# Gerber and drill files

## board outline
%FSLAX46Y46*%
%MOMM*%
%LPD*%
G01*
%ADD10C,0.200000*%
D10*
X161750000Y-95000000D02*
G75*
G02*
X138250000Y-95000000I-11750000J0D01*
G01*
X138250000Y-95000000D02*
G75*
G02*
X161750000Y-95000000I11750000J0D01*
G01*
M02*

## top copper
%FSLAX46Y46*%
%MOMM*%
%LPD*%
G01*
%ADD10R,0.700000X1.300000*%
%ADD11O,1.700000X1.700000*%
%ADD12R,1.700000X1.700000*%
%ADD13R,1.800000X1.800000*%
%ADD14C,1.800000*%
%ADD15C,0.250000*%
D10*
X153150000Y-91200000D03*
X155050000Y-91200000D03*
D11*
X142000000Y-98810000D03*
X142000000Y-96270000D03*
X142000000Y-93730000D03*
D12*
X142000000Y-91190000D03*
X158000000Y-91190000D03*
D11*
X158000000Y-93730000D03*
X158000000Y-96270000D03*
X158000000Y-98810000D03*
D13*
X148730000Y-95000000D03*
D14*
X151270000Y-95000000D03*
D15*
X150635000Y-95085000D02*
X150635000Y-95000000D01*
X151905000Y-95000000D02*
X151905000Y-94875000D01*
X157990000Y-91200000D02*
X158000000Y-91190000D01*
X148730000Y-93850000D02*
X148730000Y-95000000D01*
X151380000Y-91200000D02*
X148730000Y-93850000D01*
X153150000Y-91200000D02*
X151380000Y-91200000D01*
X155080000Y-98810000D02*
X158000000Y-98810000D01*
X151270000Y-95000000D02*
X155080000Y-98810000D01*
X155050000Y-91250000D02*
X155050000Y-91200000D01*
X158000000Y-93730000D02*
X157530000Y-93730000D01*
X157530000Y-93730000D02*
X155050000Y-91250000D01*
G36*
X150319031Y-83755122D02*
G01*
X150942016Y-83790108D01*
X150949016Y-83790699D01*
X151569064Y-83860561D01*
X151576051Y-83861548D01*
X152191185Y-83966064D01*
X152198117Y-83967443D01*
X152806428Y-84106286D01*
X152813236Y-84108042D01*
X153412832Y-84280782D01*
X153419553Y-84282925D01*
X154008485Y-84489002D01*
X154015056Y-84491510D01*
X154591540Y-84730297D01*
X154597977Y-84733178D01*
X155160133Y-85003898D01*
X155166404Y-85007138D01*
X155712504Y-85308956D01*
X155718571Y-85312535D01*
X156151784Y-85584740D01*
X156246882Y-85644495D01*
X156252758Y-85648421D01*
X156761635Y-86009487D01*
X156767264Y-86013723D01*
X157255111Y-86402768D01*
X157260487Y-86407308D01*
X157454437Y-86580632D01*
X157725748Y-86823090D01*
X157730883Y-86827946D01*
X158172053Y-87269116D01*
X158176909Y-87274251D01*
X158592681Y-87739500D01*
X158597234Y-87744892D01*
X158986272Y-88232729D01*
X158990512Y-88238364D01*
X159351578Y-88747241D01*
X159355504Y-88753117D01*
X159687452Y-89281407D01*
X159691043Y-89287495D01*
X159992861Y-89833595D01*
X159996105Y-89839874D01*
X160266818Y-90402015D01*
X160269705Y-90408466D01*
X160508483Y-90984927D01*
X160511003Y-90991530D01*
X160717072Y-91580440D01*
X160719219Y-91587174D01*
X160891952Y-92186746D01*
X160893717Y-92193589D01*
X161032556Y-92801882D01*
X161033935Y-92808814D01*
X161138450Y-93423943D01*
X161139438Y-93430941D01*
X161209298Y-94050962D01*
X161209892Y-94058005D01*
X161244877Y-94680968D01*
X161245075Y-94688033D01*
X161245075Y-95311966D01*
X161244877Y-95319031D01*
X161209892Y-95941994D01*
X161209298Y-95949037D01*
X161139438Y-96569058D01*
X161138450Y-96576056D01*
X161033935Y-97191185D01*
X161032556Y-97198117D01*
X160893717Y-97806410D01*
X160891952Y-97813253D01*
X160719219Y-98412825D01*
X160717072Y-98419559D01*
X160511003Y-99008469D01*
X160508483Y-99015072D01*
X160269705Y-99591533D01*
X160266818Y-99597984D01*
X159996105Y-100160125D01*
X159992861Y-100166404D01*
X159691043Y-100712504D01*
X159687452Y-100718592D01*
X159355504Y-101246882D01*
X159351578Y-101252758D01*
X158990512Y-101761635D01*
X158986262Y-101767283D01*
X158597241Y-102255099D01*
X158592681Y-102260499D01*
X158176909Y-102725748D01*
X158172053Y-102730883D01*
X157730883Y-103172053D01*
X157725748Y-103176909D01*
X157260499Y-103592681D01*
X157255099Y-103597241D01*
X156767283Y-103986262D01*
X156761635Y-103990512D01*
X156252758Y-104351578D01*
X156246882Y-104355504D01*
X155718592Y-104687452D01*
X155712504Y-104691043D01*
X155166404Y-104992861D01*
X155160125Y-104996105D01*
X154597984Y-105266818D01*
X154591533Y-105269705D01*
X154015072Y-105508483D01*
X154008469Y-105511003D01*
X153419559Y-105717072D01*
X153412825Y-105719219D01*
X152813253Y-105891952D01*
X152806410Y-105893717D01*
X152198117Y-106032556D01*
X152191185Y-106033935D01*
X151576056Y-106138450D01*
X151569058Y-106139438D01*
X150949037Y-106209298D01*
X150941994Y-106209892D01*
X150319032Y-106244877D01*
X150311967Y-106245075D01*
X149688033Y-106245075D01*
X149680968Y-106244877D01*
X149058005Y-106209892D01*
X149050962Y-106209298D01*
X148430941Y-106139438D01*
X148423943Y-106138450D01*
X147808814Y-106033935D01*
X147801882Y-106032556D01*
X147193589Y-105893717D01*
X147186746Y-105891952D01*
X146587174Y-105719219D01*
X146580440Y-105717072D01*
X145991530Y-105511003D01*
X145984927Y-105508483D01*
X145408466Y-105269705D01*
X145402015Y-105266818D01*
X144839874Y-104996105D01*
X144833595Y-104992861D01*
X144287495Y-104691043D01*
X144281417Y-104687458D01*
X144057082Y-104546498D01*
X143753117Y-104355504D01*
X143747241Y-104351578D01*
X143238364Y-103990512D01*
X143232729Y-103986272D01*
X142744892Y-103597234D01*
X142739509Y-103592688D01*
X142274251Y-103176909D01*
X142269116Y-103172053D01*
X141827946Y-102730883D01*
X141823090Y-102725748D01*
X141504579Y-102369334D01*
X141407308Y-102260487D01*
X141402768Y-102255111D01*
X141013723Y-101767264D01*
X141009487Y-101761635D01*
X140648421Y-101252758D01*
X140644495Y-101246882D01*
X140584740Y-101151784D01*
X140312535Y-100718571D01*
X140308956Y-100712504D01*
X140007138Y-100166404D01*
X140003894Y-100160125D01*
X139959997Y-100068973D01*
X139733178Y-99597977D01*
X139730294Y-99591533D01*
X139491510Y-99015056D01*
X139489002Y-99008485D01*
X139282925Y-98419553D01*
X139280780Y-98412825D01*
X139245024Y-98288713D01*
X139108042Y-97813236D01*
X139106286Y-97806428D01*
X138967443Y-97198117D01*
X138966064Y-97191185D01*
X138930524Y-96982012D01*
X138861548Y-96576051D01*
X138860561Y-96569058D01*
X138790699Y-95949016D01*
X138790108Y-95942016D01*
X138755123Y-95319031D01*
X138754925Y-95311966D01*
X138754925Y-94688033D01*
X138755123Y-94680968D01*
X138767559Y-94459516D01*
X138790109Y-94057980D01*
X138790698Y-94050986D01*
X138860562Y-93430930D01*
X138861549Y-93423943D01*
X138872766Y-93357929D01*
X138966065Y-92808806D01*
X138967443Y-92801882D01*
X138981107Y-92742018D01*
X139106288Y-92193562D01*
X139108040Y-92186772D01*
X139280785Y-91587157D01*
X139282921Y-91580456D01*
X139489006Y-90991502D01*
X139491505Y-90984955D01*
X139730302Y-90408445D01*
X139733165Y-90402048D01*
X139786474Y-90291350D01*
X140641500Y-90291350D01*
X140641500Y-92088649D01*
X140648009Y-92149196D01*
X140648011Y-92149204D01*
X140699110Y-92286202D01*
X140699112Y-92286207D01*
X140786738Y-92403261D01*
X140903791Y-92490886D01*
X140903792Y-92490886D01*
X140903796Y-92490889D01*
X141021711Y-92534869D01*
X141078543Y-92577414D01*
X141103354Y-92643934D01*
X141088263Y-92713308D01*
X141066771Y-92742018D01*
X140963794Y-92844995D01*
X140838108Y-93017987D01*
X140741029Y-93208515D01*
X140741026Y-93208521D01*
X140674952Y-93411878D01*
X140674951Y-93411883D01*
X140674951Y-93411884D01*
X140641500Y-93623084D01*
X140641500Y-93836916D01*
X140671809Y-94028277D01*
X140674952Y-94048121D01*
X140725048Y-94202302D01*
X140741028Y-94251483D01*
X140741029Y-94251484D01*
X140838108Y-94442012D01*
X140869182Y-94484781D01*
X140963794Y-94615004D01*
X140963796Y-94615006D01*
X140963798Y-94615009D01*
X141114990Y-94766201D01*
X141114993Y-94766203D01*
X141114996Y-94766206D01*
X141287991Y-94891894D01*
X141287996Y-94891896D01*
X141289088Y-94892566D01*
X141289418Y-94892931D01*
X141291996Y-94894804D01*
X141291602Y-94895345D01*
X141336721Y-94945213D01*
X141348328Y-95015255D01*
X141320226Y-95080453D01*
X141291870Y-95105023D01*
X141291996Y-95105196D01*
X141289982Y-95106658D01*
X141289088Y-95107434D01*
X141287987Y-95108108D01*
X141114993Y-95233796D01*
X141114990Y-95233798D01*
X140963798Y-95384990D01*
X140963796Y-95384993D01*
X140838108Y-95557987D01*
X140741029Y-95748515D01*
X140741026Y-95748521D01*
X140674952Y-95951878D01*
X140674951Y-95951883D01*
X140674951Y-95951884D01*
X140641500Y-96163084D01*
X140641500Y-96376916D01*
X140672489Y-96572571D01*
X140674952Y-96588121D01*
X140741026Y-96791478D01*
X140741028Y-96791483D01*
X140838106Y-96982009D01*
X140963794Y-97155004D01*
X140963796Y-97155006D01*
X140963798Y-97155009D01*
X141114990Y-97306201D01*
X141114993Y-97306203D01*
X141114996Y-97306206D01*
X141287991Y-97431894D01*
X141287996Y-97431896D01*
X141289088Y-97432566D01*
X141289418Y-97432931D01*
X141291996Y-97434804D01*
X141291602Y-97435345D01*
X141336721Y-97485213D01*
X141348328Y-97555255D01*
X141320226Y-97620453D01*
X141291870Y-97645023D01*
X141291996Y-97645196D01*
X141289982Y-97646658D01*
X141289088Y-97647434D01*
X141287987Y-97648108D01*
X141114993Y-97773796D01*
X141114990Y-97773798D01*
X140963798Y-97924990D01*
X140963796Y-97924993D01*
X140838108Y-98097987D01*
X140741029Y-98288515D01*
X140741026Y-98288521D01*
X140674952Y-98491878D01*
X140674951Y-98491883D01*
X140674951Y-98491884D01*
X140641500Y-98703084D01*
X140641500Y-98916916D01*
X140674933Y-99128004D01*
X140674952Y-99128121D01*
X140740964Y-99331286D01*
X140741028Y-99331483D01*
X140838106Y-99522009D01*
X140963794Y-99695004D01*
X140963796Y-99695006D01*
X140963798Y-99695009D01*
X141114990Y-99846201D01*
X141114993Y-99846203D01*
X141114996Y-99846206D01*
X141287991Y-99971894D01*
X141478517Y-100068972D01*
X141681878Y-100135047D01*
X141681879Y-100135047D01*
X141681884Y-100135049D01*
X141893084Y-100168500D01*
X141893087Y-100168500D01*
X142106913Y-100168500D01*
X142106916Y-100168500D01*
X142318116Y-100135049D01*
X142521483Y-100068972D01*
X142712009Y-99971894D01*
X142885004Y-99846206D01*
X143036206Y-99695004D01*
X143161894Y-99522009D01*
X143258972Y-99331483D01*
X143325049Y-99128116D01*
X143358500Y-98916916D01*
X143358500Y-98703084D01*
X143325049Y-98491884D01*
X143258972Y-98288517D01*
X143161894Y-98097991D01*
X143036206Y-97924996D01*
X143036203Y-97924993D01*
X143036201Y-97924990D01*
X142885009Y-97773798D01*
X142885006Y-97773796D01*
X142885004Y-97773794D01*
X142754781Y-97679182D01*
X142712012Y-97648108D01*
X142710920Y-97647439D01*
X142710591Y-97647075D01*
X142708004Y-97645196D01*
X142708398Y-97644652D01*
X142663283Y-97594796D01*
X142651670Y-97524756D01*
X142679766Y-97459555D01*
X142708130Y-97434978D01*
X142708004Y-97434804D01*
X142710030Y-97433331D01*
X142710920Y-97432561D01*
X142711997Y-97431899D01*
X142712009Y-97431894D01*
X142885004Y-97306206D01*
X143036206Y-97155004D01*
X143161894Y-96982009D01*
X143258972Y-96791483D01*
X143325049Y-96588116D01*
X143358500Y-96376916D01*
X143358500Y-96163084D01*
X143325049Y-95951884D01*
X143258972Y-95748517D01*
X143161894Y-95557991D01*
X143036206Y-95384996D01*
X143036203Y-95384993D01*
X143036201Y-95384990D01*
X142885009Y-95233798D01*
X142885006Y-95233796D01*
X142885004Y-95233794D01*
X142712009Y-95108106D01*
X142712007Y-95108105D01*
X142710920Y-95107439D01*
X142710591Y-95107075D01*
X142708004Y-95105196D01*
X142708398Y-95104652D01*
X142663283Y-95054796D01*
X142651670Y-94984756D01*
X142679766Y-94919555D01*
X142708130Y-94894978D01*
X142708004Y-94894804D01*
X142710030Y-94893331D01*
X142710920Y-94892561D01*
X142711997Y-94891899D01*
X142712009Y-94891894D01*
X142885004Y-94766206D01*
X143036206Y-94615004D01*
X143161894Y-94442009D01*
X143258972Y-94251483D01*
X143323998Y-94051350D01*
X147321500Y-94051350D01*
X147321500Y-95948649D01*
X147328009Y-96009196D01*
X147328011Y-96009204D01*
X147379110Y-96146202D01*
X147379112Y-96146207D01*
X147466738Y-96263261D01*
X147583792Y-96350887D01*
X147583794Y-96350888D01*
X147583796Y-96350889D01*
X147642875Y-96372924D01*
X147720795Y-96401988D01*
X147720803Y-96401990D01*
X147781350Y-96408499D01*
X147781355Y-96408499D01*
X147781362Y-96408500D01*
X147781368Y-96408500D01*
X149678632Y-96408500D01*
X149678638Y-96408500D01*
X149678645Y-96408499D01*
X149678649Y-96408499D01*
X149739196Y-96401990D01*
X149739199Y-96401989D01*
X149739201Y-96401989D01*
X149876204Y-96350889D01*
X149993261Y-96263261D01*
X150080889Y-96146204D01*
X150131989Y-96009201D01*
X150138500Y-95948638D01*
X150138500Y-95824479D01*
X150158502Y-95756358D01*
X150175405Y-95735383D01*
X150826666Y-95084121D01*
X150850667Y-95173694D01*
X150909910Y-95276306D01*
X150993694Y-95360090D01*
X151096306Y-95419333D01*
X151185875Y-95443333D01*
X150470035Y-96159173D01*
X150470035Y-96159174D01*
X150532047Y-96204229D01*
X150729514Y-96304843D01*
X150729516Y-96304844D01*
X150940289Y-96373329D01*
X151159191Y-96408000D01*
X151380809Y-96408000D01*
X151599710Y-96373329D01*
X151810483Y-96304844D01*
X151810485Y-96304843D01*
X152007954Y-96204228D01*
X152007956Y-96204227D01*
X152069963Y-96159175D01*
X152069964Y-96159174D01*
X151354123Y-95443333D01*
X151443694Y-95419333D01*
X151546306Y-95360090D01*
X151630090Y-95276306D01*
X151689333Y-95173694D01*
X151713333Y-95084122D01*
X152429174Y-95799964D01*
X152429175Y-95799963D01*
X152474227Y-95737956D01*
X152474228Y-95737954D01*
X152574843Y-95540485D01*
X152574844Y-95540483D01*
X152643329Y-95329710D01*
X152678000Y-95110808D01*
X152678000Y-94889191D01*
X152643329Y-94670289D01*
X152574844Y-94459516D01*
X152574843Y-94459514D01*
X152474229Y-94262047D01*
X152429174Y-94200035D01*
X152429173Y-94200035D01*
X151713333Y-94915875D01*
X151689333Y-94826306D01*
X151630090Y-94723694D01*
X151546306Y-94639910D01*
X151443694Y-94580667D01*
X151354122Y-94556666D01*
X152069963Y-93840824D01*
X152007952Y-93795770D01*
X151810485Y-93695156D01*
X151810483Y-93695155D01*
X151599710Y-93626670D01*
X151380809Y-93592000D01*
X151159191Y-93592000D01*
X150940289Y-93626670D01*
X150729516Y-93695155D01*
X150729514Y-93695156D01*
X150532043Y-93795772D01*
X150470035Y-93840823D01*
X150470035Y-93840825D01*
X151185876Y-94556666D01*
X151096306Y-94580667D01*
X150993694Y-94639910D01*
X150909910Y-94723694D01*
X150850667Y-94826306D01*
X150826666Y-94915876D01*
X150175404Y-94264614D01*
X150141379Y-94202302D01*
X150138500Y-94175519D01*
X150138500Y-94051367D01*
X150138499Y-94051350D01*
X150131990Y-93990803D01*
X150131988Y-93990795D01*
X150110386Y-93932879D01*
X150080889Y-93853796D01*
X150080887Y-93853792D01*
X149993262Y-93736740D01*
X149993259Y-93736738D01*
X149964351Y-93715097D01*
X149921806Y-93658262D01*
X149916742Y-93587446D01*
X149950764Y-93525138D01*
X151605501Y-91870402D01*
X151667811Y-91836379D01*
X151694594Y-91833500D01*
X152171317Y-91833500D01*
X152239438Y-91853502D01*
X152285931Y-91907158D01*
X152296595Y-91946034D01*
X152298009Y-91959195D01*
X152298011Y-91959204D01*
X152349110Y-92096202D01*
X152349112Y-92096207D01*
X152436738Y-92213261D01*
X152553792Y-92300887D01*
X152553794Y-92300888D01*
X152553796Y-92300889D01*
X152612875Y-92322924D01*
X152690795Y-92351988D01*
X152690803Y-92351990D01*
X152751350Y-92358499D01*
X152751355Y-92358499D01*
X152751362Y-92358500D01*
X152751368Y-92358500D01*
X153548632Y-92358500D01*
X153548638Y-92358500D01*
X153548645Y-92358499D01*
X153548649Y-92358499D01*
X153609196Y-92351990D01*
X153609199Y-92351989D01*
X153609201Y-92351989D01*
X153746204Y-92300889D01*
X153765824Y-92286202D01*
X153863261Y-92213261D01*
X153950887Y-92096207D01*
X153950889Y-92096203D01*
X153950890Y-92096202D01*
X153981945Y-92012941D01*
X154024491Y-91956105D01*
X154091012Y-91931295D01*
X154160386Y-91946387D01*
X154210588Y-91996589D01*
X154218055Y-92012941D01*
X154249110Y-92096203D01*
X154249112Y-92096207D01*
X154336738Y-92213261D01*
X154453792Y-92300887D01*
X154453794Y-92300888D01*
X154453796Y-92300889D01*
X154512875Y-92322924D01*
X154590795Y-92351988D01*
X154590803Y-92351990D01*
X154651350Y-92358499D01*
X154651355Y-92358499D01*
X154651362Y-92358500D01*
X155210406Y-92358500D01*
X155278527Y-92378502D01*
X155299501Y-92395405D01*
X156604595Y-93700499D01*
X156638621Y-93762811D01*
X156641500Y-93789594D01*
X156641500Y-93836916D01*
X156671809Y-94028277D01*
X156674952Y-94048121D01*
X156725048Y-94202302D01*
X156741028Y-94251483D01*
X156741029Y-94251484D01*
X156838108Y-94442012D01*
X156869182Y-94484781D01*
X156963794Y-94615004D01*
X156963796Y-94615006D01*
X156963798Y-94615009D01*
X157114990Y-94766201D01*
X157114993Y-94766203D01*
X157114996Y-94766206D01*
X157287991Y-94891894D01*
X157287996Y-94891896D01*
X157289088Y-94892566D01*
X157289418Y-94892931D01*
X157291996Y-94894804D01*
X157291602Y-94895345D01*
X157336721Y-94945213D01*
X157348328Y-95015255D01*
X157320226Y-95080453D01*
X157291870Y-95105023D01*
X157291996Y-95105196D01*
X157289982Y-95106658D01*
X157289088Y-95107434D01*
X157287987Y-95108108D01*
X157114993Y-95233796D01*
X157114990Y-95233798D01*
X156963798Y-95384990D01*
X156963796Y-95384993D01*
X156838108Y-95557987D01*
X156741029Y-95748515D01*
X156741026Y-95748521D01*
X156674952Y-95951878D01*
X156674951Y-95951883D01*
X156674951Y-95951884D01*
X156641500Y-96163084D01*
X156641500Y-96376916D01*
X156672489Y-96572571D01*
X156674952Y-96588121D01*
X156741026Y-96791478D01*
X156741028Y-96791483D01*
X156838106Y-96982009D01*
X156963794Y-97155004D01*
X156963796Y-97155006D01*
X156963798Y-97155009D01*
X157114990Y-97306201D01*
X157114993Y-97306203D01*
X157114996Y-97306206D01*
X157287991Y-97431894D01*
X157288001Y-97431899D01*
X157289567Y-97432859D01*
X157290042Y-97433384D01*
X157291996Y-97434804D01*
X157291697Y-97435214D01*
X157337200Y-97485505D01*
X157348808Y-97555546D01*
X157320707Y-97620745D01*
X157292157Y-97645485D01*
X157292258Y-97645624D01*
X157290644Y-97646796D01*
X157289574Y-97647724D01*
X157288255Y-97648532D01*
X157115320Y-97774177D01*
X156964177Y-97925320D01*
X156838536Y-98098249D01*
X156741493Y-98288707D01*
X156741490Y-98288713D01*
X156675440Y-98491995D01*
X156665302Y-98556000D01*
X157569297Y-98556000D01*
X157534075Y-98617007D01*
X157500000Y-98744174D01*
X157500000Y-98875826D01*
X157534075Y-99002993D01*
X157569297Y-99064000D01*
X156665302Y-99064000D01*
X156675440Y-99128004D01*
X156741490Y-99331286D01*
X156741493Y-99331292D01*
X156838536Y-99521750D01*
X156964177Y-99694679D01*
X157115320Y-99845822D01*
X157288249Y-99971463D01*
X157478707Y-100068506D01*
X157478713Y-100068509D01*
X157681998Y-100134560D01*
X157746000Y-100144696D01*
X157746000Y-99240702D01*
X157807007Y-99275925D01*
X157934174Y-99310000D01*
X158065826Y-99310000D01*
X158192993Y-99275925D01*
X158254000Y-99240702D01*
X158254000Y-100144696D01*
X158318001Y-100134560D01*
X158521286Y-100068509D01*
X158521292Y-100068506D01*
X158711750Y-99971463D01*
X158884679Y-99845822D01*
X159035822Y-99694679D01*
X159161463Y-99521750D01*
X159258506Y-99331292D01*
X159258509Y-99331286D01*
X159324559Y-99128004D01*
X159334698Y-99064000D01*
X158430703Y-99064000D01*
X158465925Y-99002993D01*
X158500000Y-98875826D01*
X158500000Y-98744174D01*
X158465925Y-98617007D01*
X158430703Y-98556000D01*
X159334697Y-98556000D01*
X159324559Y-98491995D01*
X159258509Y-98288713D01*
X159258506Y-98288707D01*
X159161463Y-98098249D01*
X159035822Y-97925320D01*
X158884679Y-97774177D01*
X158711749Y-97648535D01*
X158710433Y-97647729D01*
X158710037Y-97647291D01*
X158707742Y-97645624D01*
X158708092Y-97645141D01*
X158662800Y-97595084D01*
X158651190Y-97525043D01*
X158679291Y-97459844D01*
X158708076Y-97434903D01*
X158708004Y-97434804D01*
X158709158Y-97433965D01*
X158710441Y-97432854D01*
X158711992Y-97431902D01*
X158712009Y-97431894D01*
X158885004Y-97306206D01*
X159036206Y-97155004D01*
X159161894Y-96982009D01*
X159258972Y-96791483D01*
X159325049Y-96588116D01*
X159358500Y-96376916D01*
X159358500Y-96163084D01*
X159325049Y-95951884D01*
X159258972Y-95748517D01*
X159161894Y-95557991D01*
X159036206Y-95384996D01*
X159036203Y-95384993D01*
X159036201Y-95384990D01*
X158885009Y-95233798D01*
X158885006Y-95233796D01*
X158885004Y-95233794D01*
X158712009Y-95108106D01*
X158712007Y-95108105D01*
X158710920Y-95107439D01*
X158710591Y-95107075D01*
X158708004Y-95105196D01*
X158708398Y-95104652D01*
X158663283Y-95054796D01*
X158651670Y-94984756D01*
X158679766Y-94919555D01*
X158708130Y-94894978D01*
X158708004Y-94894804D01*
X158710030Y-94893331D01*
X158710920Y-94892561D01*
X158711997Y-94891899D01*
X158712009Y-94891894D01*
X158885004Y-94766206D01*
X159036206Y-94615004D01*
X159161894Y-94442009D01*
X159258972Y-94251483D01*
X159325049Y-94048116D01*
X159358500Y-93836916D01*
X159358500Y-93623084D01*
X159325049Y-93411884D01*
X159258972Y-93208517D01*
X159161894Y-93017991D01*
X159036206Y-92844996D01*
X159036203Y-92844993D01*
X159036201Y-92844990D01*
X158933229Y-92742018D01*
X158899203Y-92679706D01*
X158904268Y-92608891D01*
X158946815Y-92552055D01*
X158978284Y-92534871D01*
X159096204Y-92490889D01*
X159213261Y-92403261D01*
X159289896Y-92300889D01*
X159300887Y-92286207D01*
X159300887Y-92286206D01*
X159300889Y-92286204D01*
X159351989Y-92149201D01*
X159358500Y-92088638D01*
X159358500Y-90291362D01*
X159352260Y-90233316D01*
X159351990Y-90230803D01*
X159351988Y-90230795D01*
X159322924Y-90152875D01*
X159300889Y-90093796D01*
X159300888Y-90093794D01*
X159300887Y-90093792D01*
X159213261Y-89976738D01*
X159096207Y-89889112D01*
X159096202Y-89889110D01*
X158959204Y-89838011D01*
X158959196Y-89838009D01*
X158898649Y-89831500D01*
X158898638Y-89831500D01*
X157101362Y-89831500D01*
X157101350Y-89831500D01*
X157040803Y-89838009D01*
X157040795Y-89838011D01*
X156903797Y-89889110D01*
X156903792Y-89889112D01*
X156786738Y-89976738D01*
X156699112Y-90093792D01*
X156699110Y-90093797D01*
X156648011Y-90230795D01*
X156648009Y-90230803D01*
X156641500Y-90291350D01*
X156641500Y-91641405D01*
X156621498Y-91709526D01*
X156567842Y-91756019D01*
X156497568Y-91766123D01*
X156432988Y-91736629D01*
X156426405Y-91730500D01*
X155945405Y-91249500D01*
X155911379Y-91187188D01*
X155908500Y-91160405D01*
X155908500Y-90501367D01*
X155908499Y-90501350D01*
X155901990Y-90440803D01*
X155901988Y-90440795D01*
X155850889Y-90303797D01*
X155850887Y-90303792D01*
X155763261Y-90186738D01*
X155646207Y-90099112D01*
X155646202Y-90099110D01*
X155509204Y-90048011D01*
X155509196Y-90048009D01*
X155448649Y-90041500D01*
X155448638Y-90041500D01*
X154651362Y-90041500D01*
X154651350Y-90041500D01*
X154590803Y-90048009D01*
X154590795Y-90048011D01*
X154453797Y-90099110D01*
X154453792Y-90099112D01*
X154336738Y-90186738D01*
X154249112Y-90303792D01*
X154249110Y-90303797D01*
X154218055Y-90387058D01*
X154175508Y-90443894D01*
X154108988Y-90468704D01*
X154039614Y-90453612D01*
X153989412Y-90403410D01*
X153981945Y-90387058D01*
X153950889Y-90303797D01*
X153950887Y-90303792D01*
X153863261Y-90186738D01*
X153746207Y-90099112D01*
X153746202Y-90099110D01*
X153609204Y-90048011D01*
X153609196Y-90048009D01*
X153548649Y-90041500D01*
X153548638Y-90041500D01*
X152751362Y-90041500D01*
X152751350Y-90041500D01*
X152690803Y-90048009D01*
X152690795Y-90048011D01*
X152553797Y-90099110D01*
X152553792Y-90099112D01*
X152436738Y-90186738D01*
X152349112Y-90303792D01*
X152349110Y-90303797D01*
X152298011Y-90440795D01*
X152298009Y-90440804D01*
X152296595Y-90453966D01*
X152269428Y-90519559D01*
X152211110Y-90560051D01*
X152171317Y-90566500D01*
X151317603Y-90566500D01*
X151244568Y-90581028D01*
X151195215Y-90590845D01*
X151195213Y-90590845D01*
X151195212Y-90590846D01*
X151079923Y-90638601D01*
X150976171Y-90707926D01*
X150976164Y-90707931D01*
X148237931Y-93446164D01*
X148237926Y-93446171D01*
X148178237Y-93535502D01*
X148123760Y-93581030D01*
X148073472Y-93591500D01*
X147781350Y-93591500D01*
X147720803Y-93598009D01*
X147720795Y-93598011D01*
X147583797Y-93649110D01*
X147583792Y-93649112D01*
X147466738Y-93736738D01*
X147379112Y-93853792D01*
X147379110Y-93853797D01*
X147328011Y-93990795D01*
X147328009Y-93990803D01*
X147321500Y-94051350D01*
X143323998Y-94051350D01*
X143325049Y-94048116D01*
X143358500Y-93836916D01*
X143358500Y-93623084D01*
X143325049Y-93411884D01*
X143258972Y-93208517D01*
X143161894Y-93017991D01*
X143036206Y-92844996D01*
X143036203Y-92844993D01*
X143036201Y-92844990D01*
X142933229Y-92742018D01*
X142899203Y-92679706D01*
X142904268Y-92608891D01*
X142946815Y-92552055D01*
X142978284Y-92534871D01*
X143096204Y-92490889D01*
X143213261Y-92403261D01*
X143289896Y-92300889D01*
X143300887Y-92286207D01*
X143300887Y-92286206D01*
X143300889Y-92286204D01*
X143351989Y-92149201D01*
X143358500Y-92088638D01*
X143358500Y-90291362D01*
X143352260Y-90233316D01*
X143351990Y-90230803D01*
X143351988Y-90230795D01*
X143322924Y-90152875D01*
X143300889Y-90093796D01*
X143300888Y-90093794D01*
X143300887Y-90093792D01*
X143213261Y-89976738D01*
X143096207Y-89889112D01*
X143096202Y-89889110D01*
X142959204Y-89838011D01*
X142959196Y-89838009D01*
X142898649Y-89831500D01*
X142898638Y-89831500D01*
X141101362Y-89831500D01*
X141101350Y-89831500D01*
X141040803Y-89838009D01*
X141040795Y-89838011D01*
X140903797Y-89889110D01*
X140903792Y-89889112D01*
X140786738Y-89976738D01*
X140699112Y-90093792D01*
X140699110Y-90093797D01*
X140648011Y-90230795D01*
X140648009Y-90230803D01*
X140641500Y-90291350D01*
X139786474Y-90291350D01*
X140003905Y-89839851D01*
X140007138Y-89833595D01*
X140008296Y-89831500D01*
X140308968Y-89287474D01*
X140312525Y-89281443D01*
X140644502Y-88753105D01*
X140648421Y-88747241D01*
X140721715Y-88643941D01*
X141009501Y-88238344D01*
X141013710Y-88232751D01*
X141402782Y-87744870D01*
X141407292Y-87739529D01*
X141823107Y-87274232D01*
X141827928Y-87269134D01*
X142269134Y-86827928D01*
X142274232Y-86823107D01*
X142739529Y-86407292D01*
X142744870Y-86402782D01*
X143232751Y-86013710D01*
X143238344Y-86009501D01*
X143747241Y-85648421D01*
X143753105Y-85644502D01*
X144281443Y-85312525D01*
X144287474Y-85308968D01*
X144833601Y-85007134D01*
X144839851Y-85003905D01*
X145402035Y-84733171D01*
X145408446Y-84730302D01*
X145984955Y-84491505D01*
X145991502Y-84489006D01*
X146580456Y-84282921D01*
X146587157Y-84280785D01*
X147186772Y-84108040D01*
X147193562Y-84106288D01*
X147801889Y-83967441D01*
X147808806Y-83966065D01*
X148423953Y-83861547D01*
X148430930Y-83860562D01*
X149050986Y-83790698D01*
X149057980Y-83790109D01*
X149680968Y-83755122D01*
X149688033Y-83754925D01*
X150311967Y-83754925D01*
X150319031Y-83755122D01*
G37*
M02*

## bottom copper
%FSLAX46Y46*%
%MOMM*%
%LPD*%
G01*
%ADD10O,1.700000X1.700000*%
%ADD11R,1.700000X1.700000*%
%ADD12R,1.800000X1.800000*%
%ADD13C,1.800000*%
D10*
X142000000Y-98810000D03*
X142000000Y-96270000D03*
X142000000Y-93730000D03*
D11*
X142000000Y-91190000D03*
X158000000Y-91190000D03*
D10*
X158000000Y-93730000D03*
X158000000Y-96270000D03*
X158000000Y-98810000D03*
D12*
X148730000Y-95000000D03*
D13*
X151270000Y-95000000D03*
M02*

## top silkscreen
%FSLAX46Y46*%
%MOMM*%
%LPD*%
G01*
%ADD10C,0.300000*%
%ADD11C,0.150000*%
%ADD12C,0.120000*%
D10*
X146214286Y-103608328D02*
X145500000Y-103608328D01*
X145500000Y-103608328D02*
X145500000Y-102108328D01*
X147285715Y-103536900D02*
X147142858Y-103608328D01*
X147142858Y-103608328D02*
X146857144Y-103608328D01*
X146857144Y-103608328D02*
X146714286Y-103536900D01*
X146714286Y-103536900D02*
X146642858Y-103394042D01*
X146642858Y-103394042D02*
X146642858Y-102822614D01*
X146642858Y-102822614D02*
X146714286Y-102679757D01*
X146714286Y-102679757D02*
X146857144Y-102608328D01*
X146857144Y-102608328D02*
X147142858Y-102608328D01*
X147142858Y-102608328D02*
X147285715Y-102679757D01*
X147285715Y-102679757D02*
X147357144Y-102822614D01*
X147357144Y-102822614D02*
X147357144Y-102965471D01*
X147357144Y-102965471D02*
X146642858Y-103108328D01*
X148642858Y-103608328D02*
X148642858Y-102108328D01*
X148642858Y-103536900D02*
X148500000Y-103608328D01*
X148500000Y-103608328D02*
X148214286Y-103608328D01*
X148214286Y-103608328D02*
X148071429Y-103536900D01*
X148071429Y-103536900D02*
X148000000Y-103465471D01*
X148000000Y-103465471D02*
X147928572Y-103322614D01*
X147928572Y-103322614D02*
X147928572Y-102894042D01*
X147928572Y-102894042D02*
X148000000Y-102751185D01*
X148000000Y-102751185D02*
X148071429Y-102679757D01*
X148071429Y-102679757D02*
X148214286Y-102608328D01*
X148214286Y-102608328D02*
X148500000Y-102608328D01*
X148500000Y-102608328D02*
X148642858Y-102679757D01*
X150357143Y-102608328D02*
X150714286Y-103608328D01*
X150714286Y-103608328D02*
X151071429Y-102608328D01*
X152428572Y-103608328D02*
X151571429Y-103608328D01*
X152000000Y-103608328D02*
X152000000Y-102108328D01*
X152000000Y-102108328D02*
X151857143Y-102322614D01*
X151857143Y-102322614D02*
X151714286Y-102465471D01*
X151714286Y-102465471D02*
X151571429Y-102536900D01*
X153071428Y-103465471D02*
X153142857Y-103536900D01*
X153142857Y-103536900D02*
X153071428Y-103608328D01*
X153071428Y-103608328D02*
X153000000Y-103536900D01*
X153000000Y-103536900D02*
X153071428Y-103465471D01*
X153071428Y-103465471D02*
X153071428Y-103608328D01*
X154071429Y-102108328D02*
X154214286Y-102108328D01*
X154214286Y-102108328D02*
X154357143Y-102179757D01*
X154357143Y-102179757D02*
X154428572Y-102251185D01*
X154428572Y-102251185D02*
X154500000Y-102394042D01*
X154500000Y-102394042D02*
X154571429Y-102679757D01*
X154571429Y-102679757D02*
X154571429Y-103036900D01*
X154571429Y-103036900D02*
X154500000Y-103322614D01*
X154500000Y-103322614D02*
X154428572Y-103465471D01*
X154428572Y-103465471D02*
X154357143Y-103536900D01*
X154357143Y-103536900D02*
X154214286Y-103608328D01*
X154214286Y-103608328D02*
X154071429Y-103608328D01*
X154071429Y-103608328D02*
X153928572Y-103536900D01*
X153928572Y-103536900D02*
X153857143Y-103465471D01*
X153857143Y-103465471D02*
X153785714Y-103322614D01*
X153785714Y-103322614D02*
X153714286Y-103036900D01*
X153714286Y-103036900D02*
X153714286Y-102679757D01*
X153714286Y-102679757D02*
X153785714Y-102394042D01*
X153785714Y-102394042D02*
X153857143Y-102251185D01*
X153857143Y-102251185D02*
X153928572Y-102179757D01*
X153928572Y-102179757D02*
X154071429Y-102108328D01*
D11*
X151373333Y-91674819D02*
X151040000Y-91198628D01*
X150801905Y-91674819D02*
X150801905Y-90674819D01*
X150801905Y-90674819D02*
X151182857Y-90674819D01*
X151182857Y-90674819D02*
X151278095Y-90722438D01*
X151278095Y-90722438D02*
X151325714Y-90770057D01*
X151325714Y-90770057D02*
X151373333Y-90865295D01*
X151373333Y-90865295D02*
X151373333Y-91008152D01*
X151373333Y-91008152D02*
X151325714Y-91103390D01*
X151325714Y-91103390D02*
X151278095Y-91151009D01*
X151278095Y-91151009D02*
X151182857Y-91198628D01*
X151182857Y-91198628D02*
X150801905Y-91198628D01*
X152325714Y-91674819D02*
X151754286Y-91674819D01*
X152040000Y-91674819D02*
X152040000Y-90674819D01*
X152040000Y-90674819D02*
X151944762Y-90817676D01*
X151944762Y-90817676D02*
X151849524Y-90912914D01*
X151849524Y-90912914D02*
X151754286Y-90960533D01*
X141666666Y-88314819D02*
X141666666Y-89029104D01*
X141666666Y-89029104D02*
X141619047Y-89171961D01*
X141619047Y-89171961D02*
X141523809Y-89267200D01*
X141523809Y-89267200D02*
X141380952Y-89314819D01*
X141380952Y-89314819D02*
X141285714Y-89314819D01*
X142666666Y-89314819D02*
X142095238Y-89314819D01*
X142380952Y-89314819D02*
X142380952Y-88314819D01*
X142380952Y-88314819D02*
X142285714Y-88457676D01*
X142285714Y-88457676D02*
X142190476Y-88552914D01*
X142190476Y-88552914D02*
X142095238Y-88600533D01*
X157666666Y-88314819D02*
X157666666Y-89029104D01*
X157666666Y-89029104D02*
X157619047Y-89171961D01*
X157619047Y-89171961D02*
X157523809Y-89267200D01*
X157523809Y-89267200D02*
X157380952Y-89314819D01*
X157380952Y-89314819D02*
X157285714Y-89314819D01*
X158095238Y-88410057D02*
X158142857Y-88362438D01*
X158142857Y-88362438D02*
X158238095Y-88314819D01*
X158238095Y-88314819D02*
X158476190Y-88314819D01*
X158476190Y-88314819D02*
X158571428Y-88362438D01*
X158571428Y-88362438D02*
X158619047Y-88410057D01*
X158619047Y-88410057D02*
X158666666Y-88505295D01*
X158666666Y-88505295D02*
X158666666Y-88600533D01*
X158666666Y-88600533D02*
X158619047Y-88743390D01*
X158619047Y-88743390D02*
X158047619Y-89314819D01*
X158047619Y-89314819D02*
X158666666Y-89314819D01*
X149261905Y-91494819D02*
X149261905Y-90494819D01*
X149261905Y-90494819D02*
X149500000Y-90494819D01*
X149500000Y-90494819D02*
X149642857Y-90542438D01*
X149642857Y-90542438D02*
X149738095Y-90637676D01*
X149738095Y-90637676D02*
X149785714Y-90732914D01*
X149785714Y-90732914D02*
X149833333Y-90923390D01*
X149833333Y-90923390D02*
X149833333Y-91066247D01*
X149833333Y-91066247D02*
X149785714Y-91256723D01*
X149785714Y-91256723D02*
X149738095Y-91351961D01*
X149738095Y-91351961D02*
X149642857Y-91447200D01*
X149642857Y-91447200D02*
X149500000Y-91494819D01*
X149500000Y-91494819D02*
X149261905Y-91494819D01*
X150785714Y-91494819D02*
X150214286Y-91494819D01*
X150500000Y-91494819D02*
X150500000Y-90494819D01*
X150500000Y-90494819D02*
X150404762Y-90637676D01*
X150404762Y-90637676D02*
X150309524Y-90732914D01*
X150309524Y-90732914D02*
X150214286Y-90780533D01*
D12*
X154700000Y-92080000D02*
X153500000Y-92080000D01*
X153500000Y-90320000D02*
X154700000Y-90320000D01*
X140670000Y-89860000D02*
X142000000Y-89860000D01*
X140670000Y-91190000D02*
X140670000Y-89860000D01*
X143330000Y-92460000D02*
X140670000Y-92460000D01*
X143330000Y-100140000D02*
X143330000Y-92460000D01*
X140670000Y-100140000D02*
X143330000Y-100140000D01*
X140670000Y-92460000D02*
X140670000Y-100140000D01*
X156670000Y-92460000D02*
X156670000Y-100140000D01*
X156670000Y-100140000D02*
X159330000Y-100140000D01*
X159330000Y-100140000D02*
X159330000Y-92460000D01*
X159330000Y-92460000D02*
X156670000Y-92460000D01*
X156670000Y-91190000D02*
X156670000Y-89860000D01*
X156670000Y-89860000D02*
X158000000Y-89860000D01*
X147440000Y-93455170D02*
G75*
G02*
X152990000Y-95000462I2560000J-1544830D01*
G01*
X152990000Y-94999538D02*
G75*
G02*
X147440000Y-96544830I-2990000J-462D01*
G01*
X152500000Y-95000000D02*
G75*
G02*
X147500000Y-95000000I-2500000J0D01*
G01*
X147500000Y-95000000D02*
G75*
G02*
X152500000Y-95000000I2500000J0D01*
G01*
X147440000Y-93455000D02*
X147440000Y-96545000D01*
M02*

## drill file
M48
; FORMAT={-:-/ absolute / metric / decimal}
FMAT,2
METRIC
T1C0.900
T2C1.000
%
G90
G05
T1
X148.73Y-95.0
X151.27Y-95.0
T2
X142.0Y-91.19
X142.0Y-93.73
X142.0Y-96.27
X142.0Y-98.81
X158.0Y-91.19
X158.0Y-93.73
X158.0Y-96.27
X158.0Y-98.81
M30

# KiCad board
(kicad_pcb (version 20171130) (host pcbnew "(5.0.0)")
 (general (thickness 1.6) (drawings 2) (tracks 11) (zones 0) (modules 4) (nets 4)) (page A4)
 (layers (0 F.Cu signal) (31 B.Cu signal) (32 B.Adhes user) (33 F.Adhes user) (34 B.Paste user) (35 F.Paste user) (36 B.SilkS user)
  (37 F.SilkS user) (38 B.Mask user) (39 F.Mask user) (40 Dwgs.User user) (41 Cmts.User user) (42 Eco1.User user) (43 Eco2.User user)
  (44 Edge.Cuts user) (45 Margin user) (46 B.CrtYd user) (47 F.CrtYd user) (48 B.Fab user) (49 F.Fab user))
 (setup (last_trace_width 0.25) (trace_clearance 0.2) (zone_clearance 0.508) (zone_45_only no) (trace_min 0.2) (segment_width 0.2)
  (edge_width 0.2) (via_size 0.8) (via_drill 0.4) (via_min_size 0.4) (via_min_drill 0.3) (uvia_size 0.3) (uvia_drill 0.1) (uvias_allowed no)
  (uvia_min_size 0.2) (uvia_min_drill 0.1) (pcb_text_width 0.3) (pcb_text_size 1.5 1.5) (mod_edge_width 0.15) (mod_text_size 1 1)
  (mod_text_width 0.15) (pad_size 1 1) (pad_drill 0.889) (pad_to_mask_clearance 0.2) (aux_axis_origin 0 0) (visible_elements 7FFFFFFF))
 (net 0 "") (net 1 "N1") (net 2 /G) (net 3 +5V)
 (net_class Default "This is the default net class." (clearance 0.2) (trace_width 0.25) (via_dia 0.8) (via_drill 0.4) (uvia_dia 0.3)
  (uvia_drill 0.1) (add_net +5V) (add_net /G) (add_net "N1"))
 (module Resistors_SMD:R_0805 (layer F.Cu) (at 154.1 91.2)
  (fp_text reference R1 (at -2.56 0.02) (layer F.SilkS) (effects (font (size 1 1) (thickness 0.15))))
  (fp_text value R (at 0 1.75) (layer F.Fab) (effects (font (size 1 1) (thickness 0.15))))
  (fp_line (start 0.6 0.88) (end -0.6 0.88) (layer F.SilkS) (width 0.12))
  (fp_line (start -0.6 -0.88) (end 0.6 -0.88) (layer F.SilkS) (width 0.12))
  (pad 1 smd rect (at -0.95 0) (size 0.7 1.3) (layers F.Cu F.Paste F.Mask) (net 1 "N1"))
  (pad 2 smd rect (at 0.95 0) (size 0.7 1.3) (layers F.Cu F.Paste F.Mask) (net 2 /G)))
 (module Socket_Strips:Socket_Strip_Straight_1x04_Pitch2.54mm (layer F.Cu) (at 142 91.19)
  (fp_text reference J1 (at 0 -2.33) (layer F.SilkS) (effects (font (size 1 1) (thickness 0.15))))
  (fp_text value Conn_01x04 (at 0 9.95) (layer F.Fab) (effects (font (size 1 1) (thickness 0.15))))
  (fp_line (start -1.33 -1.33) (end 0 -1.33) (layer F.SilkS) (width 0.12))
  (fp_line (start -1.33 0) (end -1.33 -1.33) (layer F.SilkS) (width 0.12))
  (fp_line (start 1.33 1.27) (end -1.33 1.27) (layer F.SilkS) (width 0.12))
  (fp_line (start 1.33 8.95) (end 1.33 1.27) (layer F.SilkS) (width 0.12))
  (fp_line (start -1.33 8.95) (end 1.33 8.95) (layer F.SilkS) (width 0.12))
  (fp_line (start -1.33 1.27) (end -1.33 8.95) (layer F.SilkS) (width 0.12))
  (pad 4 thru_hole oval (at 0 7.62) (size 1.7 1.7) (drill 1) (layers *.Cu *.Mask))
  (pad 3 thru_hole oval (at 0 5.08) (size 1.7 1.7) (drill 1) (layers *.Cu *.Mask))
  (pad 2 thru_hole oval (at 0 2.54) (size 1.7 1.7) (drill 1) (layers *.Cu *.Mask))
  (pad 1 thru_hole rect (at 0 0) (size 1.7 1.7) (drill 1) (layers *.Cu *.Mask)))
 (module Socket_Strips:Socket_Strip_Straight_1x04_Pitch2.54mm (layer F.Cu) (at 158 91.19)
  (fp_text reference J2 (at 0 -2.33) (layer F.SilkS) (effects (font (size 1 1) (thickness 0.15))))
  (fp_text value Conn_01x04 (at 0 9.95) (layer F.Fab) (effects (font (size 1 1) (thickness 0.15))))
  (fp_line (start -1.33 1.27) (end -1.33 8.95) (layer F.SilkS) (width 0.12))
  (fp_line (start -1.33 8.95) (end 1.33 8.95) (layer F.SilkS) (width 0.12))
  (fp_line (start 1.33 8.95) (end 1.33 1.27) (layer F.SilkS) (width 0.12))
  (fp_line (start 1.33 1.27) (end -1.33 1.27) (layer F.SilkS) (width 0.12))
  (fp_line (start -1.33 0) (end -1.33 -1.33) (layer F.SilkS) (width 0.12))
  (fp_line (start -1.33 -1.33) (end 0 -1.33) (layer F.SilkS) (width 0.12))
  (pad 1 thru_hole rect (at 0 0) (size 1.7 1.7) (drill 1) (layers *.Cu *.Mask))
  (pad 2 thru_hole oval (at 0 2.54) (size 1.7 1.7) (drill 1) (layers *.Cu *.Mask) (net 2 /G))
  (pad 3 thru_hole oval (at 0 5.08) (size 1.7 1.7) (drill 1) (layers *.Cu *.Mask))
  (pad 4 thru_hole oval (at 0 7.62) (size 1.7 1.7) (drill 1) (layers *.Cu *.Mask) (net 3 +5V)))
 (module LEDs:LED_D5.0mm (layer F.Cu) (at 148.73 95)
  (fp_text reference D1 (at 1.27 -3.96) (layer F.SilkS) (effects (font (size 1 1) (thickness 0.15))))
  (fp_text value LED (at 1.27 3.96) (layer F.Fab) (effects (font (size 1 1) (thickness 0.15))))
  (fp_arc (start 1.27 0) (end -1.29 -1.54483) (angle 148.9) (layer F.SilkS) (width 0.12))
  (fp_arc (start 1.27 0) (end -1.29 1.54483) (angle -148.9) (layer F.SilkS) (width 0.12))
  (fp_circle (center 1.27 0) (end 3.77 0) (layer F.SilkS) (width 0.12))
  (fp_line (start -1.29 -1.545) (end -1.29 1.545) (layer F.SilkS) (width 0.12))
  (pad 1 thru_hole rect (at 0 0) (size 1.8 1.8) (drill 0.9) (layers *.Cu *.Mask) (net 1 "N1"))
  (pad 2 thru_hole circle (at 2.54 0) (size 1.8 1.8) (drill 0.9) (layers *.Cu *.Mask) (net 3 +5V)))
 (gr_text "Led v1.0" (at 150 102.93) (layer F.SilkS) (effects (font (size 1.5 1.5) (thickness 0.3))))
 (gr_circle (center 150 95) (end 161.75 95) (layer Edge.Cuts) (width 0.2))
 (segment (start 150.635 95.085) (end 150.635 95) (width 0.25) (layer F.Cu) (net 3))
 (segment (start 151.905 95) (end 151.905 94.875) (width 0.25) (layer F.Cu) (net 3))
 (segment (start 157.99 91.2) (end 158 91.19) (width 0.25) (layer F.Cu) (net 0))
 (segment (start 148.73 93.85) (end 148.73 95) (width 0.25) (layer F.Cu) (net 1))
 (segment (start 151.38 91.2) (end 148.73 93.85) (width 0.25) (layer F.Cu) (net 1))
 (segment (start 153.15 91.2) (end 151.38 91.2) (width 0.25) (layer F.Cu) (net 1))
 (segment (start 155.08 98.81) (end 158 98.81) (width 0.25) (layer F.Cu) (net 3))
 (segment (start 151.27 95) (end 155.08 98.81) (width 0.25) (layer F.Cu) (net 3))
 (segment (start 155.05 91.25) (end 155.05 91.2) (width 0.25) (layer F.Cu) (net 2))
 (segment (start 158 93.73) (end 157.53 93.73) (width 0.25) (layer F.Cu) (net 2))
 (segment (start 157.53 93.73) (end 155.05 91.25) (width 0.25) (layer F.Cu) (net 2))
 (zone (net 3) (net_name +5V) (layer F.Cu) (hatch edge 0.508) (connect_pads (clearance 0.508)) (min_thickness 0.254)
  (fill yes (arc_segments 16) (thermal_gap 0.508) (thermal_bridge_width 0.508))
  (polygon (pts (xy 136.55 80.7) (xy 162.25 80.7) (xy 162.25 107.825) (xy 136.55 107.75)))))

